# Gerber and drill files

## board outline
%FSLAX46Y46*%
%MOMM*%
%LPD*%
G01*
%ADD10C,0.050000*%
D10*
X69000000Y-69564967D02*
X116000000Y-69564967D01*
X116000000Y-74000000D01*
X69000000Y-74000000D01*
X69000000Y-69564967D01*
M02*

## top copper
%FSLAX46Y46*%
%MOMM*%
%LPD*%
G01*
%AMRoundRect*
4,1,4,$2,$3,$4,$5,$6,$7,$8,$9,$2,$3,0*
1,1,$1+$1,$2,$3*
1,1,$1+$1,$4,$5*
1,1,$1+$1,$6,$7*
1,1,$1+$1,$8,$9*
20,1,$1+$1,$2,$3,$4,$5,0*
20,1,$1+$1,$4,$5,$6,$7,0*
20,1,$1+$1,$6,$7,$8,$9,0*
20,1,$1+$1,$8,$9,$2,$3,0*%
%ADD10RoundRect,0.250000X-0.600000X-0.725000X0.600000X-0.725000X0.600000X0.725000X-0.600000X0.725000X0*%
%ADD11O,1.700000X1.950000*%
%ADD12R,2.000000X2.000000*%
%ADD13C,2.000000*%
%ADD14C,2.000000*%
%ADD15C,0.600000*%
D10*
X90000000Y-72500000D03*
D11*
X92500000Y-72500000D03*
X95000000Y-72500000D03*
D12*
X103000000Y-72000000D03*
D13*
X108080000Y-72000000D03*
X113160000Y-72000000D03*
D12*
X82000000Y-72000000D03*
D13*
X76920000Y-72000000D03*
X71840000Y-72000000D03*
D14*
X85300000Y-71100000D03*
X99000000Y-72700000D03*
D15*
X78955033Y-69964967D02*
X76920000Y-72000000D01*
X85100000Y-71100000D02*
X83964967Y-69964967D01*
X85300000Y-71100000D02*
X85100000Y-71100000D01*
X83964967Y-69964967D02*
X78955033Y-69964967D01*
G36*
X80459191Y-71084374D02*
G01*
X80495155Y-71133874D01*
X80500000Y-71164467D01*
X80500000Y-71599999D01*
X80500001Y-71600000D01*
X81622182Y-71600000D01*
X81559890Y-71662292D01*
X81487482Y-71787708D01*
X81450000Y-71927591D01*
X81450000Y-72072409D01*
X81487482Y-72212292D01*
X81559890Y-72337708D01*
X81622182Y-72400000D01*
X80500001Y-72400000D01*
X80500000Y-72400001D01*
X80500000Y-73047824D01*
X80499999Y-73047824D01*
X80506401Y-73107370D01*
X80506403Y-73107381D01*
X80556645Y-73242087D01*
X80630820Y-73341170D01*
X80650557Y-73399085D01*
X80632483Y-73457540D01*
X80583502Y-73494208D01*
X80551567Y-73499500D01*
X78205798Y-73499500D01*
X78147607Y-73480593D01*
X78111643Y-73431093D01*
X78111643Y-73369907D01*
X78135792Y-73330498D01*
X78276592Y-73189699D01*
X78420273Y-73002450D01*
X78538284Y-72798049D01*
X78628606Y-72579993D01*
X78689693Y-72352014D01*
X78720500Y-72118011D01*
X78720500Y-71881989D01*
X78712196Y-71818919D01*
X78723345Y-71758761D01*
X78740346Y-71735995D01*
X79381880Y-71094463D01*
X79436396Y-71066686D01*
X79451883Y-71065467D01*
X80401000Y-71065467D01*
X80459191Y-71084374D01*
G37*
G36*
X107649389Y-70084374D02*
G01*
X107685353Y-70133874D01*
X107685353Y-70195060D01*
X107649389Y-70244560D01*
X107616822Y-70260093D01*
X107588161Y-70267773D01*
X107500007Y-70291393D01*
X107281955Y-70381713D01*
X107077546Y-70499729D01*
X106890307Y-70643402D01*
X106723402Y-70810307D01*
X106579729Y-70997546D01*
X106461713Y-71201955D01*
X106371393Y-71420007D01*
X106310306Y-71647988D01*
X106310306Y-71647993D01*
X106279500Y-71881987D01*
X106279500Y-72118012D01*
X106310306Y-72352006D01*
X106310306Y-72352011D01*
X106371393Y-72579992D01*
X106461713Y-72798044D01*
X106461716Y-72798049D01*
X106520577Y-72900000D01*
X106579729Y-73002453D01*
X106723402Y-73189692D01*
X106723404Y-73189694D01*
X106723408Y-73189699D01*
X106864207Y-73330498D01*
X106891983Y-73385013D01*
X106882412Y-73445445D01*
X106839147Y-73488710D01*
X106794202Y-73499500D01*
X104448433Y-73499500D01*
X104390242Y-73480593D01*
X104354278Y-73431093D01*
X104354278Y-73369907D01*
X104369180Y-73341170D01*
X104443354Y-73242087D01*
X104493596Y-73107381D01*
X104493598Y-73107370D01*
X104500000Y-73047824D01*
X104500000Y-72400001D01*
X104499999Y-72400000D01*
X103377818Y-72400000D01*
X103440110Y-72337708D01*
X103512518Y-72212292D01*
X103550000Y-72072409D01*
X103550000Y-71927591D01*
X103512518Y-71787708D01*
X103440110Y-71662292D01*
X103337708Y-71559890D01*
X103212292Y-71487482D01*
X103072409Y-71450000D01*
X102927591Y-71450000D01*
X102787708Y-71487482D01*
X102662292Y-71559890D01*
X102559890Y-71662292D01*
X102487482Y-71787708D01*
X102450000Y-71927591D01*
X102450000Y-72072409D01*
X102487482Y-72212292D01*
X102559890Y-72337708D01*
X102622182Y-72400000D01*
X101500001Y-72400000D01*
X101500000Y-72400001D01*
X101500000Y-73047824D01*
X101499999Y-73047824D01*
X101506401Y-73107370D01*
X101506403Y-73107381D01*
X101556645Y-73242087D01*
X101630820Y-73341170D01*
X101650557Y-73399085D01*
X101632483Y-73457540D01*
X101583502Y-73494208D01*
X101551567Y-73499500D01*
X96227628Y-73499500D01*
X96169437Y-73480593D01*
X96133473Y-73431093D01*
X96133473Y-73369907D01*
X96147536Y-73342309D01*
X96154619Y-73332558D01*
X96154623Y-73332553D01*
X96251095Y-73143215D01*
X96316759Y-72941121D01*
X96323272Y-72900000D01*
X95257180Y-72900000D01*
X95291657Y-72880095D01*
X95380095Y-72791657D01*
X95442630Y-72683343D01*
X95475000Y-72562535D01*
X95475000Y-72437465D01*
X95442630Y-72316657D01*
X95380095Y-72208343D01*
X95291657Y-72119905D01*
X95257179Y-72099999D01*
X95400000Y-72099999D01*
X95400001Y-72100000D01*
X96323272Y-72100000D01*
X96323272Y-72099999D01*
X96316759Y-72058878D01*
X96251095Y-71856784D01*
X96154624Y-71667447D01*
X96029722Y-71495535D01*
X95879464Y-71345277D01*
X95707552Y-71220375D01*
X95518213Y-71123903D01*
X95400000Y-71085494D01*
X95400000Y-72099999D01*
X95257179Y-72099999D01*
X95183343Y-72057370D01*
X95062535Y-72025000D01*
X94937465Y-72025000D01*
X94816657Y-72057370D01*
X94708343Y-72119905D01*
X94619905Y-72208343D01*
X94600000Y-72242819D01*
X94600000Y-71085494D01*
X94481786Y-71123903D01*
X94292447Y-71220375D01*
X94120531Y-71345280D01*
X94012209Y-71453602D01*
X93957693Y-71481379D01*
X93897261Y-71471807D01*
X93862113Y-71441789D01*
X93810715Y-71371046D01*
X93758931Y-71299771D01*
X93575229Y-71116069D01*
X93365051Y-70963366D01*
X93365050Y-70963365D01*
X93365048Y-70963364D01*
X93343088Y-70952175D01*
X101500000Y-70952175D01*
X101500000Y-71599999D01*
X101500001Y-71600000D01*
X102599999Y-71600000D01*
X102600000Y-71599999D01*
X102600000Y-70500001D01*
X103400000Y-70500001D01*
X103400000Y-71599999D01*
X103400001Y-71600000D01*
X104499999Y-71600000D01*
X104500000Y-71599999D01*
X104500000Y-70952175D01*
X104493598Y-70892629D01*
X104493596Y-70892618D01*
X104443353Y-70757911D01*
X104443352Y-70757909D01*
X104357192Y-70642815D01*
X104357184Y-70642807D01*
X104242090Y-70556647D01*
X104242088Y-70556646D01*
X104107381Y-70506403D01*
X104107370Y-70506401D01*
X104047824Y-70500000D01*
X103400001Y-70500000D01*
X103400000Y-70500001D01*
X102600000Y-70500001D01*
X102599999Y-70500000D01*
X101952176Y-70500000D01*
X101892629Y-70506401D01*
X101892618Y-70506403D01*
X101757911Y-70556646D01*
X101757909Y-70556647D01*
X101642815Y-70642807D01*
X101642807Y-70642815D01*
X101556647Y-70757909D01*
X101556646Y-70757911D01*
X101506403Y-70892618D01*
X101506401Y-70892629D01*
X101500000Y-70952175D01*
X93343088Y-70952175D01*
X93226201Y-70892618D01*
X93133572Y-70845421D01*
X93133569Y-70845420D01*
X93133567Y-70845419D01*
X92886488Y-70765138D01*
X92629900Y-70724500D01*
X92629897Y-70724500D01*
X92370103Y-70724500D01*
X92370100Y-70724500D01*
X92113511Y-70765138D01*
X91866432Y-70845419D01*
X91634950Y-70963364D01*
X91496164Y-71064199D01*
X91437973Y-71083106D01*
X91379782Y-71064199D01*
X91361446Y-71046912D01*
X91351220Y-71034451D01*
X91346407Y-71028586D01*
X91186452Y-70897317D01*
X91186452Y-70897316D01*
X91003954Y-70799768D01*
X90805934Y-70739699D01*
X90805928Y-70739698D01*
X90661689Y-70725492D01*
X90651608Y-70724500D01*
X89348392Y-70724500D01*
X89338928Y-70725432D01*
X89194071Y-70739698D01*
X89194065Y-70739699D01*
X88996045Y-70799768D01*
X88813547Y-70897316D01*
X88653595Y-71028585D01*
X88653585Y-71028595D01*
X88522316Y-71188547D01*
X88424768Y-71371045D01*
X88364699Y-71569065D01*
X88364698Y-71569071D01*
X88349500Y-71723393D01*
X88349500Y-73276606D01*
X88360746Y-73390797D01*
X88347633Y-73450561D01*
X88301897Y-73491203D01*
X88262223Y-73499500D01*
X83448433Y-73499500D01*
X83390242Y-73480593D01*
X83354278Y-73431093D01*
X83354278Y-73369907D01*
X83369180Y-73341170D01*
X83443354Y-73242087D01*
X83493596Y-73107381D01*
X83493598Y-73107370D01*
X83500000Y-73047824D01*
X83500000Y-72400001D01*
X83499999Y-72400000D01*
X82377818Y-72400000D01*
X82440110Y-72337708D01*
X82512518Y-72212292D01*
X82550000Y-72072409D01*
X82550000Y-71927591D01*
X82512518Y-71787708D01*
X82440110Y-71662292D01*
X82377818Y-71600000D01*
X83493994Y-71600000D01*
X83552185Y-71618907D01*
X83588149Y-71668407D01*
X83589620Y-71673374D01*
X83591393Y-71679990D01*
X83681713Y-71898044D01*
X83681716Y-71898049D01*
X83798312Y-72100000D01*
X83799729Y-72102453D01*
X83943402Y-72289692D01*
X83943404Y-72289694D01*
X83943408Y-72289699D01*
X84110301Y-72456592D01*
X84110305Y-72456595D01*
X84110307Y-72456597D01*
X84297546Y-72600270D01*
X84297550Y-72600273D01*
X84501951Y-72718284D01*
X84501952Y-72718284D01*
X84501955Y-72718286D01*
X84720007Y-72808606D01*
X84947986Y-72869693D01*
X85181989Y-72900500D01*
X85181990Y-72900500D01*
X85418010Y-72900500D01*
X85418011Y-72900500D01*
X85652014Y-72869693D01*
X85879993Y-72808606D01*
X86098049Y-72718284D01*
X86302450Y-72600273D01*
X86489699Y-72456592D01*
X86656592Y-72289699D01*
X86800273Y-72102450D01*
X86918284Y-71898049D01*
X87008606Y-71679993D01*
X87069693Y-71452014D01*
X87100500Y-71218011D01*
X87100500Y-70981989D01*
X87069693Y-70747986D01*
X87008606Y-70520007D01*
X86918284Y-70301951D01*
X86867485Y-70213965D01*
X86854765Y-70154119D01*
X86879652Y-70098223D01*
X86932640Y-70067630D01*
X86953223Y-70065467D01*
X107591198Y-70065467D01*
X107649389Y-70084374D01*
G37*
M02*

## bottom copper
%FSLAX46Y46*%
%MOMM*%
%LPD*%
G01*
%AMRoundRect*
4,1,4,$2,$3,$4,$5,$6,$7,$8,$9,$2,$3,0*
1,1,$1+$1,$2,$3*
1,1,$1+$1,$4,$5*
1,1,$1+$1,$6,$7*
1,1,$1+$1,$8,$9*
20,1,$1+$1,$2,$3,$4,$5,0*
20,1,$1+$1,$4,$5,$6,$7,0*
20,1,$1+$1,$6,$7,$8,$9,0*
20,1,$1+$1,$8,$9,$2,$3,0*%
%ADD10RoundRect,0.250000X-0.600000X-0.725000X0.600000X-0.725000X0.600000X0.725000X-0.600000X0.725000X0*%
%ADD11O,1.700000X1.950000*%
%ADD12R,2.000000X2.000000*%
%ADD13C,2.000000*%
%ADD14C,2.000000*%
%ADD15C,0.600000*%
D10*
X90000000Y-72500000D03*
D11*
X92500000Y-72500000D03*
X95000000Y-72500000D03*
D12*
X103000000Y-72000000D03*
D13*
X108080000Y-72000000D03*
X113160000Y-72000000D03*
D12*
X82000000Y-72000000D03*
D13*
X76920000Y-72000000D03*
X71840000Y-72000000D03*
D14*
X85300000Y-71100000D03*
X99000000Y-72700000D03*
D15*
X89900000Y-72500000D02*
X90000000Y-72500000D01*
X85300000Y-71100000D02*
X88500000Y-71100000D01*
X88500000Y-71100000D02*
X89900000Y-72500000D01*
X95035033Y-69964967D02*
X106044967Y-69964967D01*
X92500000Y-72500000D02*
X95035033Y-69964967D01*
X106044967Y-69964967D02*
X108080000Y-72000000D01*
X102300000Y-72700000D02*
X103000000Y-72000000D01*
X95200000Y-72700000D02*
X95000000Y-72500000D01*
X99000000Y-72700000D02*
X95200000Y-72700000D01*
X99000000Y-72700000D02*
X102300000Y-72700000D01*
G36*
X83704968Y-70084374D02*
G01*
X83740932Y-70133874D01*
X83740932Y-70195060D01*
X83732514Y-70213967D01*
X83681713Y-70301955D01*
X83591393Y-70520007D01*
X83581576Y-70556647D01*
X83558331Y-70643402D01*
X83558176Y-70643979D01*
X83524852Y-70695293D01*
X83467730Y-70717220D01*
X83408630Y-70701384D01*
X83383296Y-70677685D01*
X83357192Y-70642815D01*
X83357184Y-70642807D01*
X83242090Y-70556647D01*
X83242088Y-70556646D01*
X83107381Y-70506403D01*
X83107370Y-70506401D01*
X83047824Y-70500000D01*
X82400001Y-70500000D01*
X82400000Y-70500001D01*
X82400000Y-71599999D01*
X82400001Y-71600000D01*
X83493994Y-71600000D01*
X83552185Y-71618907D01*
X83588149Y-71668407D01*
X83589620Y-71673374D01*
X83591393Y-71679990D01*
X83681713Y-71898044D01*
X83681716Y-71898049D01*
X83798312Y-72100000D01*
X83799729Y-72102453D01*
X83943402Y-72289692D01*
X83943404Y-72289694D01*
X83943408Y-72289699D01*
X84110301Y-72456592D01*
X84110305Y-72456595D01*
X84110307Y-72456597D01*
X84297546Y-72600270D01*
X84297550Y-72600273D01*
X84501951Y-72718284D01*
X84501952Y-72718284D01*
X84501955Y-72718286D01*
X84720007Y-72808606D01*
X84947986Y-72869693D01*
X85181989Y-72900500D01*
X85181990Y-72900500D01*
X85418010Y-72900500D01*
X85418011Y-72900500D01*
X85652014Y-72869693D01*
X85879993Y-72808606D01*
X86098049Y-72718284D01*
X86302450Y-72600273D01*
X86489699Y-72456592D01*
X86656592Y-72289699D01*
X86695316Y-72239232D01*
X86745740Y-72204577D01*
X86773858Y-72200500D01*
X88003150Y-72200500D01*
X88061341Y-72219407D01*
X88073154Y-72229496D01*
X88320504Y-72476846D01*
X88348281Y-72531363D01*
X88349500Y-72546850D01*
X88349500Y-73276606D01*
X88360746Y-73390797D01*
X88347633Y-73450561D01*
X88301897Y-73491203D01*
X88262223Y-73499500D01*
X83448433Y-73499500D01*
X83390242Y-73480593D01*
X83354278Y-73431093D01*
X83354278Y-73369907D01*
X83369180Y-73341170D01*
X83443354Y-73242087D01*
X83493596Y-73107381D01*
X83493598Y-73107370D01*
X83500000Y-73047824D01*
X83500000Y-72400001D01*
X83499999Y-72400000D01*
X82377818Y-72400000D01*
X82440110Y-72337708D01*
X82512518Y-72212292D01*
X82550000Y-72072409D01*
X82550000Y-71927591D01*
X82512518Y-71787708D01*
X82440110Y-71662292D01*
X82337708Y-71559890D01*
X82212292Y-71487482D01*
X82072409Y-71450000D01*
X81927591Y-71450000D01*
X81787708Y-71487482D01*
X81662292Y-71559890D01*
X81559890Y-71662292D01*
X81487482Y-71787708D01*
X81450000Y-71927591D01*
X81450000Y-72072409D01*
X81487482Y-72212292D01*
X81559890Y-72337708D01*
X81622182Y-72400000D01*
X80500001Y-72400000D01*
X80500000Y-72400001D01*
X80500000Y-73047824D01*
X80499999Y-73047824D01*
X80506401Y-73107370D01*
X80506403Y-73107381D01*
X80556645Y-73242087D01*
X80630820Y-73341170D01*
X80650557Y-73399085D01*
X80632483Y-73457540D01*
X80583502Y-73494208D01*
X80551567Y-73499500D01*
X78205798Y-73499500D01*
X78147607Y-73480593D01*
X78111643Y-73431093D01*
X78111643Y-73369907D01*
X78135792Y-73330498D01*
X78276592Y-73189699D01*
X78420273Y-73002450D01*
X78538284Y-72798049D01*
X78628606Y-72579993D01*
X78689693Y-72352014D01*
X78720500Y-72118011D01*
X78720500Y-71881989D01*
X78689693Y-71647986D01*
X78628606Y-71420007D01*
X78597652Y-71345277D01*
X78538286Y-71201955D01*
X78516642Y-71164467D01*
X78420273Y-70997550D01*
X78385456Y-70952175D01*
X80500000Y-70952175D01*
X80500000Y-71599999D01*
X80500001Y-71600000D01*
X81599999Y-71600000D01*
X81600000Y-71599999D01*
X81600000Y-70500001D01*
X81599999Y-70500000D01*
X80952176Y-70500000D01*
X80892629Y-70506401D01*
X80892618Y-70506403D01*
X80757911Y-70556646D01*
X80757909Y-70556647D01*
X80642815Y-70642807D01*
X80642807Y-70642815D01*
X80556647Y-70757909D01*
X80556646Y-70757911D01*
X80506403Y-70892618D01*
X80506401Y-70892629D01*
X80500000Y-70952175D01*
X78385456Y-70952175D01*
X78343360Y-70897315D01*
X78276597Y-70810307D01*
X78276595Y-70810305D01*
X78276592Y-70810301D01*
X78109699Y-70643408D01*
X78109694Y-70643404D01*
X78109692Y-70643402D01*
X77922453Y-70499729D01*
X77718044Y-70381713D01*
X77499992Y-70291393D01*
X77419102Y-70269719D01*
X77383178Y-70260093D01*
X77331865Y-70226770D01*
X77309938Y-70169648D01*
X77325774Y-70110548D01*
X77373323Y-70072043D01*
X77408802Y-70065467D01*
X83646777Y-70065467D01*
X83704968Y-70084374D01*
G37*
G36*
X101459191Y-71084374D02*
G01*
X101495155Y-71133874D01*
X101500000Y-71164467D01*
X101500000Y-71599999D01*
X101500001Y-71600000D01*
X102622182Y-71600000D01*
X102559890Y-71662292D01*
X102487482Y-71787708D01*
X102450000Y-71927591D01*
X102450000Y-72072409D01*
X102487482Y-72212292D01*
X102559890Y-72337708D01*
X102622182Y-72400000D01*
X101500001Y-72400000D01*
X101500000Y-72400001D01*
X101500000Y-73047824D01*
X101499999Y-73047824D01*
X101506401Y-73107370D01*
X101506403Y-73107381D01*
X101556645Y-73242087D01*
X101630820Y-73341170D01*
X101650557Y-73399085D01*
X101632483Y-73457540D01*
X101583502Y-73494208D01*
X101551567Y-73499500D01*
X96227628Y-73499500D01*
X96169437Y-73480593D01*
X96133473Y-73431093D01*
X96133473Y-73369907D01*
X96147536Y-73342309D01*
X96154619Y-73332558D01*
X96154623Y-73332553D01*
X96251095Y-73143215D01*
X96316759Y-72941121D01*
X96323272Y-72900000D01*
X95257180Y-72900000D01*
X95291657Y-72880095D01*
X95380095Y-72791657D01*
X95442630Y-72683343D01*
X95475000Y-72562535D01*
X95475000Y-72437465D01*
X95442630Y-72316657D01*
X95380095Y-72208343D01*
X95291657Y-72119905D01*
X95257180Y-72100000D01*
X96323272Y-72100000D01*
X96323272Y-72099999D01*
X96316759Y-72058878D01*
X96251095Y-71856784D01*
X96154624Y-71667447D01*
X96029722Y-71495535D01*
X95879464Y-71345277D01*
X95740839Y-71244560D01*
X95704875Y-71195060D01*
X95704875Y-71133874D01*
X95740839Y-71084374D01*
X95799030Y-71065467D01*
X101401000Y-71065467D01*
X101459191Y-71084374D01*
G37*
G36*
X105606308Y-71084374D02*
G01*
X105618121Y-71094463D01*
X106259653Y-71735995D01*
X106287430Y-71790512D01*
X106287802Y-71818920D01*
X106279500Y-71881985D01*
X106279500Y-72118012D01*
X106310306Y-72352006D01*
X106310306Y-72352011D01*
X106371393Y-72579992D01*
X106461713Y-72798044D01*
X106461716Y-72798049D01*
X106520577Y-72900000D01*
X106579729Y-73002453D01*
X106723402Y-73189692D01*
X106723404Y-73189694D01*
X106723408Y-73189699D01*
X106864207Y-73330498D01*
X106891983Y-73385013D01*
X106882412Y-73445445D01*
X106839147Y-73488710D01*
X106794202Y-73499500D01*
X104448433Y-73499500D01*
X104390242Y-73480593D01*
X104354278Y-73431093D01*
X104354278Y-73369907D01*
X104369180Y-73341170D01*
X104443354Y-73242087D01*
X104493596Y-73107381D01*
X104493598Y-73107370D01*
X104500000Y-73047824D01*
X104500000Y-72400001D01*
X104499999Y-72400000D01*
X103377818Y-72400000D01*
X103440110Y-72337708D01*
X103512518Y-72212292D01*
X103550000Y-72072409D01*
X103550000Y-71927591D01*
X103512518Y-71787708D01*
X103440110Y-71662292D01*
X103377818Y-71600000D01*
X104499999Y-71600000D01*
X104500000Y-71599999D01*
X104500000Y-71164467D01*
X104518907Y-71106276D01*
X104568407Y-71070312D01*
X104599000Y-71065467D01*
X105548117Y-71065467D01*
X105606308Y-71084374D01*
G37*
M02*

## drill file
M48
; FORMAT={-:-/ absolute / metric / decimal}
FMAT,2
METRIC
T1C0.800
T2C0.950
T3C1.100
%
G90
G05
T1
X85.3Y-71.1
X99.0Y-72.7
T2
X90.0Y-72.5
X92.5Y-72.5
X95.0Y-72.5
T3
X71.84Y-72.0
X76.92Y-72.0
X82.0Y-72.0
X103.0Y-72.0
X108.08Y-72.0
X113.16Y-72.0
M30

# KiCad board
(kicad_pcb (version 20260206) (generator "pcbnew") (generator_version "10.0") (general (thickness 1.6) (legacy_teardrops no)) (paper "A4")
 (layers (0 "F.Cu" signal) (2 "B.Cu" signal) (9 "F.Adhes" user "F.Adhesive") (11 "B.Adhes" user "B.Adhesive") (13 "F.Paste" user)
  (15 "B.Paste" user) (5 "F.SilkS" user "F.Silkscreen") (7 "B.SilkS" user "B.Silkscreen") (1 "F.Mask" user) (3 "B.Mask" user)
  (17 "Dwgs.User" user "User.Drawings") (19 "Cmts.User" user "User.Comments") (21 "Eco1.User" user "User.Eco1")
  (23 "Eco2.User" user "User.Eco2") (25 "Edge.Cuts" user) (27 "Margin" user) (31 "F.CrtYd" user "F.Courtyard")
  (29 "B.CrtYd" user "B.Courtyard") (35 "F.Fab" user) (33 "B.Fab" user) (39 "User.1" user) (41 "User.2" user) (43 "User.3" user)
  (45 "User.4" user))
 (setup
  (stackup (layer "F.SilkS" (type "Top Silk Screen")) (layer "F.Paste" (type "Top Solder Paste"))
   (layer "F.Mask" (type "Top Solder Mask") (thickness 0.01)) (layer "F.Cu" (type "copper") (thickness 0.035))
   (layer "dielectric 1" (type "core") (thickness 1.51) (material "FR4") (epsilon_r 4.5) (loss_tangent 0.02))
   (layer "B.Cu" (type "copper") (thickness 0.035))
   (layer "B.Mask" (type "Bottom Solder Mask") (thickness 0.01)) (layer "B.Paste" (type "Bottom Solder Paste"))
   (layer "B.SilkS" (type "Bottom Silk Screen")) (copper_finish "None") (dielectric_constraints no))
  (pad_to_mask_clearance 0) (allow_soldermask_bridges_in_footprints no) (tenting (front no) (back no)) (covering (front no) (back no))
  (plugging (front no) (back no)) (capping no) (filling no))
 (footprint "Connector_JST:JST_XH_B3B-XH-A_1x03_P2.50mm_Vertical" (layer "F.Cu") (at 90 72.5)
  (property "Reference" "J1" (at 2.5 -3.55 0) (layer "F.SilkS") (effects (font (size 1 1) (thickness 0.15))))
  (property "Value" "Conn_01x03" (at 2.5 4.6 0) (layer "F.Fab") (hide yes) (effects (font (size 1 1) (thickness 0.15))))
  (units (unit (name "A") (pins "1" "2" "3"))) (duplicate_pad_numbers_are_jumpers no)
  (pad "1" thru_hole roundrect (at 0 0) (size 1.7 1.95) (drill 0.95) (layers "*.Cu" "*.Mask") (remove_unused_layers no)
   (roundrect_rratio 0.147059) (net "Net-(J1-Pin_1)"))
  (pad "2" thru_hole oval (at 2.5 0) (size 1.7 1.95) (drill 0.95) (layers "*.Cu" "*.Mask") (remove_unused_layers no) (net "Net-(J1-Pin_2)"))
  (pad "3" thru_hole oval (at 5 0) (size 1.7 1.95) (drill 0.95) (layers "*.Cu" "*.Mask") (remove_unused_layers no) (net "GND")))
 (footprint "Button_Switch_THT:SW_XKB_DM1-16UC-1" (layer "F.Cu") (at 103 72)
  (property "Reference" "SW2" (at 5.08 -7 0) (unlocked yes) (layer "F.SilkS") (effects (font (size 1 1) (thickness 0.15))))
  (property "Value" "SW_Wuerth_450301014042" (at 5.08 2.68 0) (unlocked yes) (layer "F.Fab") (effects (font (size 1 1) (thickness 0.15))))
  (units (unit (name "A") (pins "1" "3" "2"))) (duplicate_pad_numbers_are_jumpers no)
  (pad "1" thru_hole rect (at 0 0) (size 2 2) (drill 1.1) (layers "*.Cu" "*.Mask") (remove_unused_layers no) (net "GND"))
  (pad "2" thru_hole circle (at 5.08 0) (size 2 2) (drill 1.1) (layers "*.Cu" "*.Mask") (remove_unused_layers no) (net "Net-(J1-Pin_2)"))
  (pad "3" thru_hole circle (at 10.16 0) (size 2 2) (drill 1.1) (layers "*.Cu" "*.Mask") (remove_unused_layers no)
   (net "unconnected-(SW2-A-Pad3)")))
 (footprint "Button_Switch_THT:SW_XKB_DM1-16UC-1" (layer "B.Cu") (at 82 72 180)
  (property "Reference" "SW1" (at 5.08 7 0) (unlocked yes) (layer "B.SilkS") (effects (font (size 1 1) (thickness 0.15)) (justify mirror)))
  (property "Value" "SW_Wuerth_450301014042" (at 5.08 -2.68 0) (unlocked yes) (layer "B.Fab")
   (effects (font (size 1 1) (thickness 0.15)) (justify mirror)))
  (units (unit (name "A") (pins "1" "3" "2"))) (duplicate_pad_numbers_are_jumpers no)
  (pad "1" thru_hole rect (at 0 0 180) (size 2 2) (drill 1.1) (layers "*.Cu" "*.Mask") (remove_unused_layers no) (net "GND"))
  (pad "2" thru_hole circle (at 5.08 0 180) (size 2 2) (drill 1.1) (layers "*.Cu" "*.Mask") (remove_unused_layers no) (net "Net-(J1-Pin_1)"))
  (pad "3" thru_hole circle (at 10.16 0 180) (size 2 2) (drill 1.1) (layers "*.Cu" "*.Mask") (remove_unused_layers no)
   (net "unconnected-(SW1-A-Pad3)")))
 (gr_rect (start 69 69.564967) (end 116 74) (stroke (width 0.05) (type default)) (fill no) (layer "Edge.Cuts"))
 (segment (start 78.955033 69.964967) (end 76.92 72) (width 0.6) (layer "F.Cu") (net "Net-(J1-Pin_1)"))
 (segment (start 85.1 71.1) (end 83.964967 69.964967) (width 0.6) (layer "F.Cu") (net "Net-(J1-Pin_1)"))
 (segment (start 85.3 71.1) (end 85.1 71.1) (width 0.6) (layer "F.Cu") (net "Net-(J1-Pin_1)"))
 (segment (start 83.964967 69.964967) (end 78.955033 69.964967) (width 0.6) (layer "F.Cu") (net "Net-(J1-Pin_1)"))
 (via (at 85.3 71.1) (size 2) (drill 0.8) (layers "F.Cu" "B.Cu") (free yes) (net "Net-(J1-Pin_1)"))
 (segment (start 89.9 72.5) (end 90 72.5) (width 0.6) (layer "B.Cu") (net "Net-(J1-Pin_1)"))
 (segment (start 85.3 71.1) (end 88.5 71.1) (width 0.6) (layer "B.Cu") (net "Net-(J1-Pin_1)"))
 (segment (start 88.5 71.1) (end 89.9 72.5) (width 0.6) (layer "B.Cu") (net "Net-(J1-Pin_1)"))
 (segment (start 95.035033 69.964967) (end 106.044967 69.964967) (width 0.6) (layer "B.Cu") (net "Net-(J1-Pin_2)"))
 (segment (start 92.5 72.5) (end 95.035033 69.964967) (width 0.6) (layer "B.Cu") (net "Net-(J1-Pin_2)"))
 (segment (start 106.044967 69.964967) (end 108.08 72) (width 0.6) (layer "B.Cu") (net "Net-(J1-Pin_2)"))
 (via (at 99 72.7) (size 2) (drill 0.8) (layers "F.Cu" "B.Cu") (free yes) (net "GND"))
 (segment (start 102.3 72.7) (end 103 72) (width 0.6) (layer "B.Cu") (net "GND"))
 (segment (start 95.2 72.7) (end 95 72.5) (width 0.6) (layer "B.Cu") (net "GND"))
 (segment (start 99 72.7) (end 95.2 72.7) (width 0.6) (layer "B.Cu") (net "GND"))
 (segment (start 99 72.7) (end 102.3 72.7) (width 0.6) (layer "B.Cu") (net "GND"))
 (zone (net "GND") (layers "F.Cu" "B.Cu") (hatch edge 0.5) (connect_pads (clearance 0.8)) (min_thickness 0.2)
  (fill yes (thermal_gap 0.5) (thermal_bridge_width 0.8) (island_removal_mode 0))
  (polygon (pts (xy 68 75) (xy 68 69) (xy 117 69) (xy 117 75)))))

